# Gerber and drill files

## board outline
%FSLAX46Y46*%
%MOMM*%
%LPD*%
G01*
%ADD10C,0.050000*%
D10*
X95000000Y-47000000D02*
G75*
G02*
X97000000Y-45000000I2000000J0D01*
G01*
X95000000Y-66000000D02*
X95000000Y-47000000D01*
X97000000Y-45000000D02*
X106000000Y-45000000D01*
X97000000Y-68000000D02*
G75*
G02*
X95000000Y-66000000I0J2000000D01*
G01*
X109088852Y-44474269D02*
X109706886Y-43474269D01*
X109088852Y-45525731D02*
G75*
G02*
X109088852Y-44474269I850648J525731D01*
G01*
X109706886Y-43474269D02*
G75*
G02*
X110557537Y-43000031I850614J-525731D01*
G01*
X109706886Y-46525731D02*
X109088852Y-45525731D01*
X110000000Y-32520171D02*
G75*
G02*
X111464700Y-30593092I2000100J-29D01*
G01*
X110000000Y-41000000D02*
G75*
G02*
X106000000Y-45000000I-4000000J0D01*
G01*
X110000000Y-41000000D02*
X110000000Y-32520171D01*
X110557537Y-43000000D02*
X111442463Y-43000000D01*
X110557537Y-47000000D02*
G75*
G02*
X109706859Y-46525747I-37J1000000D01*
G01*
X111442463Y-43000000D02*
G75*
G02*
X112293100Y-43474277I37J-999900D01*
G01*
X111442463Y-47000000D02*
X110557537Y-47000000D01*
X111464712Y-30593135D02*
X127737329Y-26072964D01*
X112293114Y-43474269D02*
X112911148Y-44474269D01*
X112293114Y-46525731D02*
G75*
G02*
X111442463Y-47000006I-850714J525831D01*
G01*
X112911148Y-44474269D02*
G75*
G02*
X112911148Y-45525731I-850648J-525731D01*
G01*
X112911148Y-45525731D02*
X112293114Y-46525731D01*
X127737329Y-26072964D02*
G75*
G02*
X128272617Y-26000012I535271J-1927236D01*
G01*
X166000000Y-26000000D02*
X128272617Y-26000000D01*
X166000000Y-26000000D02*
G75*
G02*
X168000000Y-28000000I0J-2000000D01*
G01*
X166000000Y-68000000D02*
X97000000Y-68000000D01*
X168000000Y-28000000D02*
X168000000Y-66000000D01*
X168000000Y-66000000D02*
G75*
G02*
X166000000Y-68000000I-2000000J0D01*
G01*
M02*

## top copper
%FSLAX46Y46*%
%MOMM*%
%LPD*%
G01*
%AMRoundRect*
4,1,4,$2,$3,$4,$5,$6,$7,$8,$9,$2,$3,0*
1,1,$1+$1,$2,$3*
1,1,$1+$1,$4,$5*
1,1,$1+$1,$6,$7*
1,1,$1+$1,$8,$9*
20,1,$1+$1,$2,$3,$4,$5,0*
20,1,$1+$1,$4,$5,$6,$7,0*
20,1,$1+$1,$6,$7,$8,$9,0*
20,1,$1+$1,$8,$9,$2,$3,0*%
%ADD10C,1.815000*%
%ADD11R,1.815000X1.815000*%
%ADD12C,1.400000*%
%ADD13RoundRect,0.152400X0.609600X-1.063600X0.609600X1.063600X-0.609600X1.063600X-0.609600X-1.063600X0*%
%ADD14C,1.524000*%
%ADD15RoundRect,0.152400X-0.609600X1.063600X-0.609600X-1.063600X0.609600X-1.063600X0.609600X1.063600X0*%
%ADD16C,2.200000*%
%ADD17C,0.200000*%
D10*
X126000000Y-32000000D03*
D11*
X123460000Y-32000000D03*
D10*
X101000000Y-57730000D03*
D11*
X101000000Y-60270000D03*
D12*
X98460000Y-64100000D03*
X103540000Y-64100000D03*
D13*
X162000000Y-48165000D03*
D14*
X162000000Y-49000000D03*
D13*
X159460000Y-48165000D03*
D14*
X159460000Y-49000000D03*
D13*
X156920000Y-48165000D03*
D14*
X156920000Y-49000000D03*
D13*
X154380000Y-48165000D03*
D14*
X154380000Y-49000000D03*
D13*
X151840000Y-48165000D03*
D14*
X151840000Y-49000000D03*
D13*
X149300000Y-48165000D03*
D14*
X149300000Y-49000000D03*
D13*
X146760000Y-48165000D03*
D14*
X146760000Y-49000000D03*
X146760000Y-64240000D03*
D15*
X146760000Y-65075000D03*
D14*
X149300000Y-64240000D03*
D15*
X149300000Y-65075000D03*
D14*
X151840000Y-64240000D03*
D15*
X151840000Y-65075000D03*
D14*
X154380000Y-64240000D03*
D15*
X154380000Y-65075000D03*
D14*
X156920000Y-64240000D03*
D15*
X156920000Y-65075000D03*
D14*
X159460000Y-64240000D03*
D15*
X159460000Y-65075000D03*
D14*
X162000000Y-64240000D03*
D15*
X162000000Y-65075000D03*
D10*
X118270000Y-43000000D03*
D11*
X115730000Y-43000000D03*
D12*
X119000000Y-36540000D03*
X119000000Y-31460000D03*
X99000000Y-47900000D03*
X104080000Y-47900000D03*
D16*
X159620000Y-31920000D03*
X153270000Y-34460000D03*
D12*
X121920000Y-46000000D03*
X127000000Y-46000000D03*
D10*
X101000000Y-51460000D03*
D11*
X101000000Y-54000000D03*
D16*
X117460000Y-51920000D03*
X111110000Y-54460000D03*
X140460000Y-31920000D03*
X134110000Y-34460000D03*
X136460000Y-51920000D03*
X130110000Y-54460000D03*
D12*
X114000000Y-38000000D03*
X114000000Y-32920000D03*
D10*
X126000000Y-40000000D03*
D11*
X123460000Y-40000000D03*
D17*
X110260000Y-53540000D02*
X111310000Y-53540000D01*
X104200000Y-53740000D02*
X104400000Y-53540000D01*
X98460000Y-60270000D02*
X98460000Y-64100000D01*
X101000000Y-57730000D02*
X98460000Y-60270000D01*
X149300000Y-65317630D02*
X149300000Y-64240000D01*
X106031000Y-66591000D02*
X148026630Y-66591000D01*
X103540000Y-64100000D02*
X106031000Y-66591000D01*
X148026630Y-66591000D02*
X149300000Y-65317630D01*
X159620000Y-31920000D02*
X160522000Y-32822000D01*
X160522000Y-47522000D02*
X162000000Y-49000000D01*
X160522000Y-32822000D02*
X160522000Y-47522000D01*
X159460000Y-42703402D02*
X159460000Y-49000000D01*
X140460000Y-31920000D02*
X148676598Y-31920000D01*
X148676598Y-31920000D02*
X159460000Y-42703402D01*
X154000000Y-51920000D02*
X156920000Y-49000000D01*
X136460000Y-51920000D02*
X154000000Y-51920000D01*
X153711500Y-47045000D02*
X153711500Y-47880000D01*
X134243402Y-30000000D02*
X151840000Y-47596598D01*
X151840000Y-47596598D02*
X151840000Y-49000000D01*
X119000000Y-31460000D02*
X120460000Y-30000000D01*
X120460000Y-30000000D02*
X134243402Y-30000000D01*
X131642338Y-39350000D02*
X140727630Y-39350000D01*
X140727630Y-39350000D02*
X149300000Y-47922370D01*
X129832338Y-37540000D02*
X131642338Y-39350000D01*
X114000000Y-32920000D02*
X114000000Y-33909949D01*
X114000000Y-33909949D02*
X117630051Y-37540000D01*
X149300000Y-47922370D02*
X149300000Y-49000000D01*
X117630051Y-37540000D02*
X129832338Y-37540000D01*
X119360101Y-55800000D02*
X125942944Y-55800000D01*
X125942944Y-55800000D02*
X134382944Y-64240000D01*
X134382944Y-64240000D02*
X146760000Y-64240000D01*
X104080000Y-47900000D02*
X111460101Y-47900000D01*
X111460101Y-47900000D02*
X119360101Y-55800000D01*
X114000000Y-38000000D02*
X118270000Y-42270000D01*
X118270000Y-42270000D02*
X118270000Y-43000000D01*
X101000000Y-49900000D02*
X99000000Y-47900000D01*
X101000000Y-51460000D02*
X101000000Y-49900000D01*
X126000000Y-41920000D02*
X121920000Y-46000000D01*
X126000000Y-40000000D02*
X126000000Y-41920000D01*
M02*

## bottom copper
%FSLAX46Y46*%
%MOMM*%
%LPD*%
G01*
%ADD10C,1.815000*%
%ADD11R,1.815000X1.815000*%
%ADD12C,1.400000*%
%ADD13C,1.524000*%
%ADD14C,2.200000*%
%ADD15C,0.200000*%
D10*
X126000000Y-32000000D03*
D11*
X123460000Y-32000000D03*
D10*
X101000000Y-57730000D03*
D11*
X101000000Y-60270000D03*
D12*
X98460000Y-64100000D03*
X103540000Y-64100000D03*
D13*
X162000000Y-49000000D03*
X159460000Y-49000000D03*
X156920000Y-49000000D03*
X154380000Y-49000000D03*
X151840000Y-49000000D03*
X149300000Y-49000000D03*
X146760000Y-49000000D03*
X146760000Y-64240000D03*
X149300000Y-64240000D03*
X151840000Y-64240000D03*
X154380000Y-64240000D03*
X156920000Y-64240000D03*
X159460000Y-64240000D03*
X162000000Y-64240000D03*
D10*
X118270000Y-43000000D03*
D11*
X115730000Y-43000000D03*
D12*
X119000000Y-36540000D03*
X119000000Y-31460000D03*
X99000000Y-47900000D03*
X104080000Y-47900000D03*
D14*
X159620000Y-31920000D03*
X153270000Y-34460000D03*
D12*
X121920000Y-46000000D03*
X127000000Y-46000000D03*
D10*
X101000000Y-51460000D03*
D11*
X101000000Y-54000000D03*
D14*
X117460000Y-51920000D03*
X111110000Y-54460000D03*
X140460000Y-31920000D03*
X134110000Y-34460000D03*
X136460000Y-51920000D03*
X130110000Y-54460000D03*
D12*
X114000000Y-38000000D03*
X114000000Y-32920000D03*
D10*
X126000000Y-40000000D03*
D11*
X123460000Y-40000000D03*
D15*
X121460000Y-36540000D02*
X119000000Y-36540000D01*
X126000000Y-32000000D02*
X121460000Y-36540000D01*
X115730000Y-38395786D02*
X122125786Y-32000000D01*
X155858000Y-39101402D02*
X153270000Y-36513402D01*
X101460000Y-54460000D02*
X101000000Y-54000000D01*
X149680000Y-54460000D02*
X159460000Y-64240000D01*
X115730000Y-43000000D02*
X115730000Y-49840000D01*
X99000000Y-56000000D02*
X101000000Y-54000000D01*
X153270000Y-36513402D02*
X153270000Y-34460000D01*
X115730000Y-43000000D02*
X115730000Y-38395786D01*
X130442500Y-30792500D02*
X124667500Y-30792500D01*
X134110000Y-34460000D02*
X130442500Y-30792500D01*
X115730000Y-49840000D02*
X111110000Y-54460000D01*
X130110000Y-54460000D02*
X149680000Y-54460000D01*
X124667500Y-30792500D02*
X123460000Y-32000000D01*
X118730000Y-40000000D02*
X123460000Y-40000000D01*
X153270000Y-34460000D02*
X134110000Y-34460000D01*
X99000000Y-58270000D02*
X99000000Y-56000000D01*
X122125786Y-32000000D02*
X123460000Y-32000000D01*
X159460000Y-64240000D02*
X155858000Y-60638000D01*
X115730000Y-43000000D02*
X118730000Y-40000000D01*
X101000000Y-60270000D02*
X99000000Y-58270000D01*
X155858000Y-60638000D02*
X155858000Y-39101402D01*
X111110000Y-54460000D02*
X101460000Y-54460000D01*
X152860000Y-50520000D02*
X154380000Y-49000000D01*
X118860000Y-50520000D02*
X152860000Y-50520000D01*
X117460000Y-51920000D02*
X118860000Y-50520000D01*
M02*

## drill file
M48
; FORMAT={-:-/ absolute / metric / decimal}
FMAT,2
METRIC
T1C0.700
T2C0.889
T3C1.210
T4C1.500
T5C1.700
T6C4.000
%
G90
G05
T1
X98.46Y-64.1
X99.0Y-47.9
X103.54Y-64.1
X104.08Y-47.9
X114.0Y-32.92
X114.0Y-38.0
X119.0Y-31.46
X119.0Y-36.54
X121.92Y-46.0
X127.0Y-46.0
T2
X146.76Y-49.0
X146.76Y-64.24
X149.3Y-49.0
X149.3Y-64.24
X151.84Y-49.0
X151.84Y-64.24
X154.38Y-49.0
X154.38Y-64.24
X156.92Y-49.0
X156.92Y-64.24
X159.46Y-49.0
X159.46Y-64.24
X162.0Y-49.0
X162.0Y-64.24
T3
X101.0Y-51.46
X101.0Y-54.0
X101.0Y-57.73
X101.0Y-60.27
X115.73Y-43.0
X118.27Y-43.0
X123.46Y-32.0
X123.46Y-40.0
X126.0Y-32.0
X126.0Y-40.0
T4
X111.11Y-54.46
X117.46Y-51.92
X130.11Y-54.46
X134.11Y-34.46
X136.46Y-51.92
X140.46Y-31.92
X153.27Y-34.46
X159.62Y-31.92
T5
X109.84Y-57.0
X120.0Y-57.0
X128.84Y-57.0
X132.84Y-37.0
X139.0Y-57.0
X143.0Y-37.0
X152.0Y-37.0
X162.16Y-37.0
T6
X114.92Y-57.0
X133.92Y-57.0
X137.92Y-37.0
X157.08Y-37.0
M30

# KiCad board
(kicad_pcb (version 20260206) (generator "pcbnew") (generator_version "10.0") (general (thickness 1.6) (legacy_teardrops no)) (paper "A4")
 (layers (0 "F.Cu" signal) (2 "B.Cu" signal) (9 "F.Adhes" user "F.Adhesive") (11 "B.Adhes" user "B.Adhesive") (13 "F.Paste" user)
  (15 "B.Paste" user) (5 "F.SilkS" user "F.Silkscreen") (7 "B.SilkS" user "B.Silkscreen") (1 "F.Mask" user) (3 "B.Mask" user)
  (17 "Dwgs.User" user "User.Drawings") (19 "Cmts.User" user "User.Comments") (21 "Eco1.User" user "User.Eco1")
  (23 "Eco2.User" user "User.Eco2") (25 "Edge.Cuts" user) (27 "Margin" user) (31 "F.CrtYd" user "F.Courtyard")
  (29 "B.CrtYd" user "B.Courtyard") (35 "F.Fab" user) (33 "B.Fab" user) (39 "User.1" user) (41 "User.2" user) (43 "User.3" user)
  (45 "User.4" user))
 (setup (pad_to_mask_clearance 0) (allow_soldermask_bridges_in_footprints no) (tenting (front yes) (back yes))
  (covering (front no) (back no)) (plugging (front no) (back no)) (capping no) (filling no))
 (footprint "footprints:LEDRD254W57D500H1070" (layer "F.Cu") (at 124.73 32)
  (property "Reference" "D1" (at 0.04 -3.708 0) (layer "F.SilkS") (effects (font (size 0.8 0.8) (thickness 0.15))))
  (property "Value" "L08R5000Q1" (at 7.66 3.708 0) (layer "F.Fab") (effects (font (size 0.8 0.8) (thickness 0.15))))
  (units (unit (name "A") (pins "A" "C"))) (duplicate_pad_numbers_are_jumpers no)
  (pad "A" thru_hole circle (at 1.27 0) (size 1.815 1.815) (drill 1.21) (layers "*.Cu" "*.Mask") (remove_unused_layers no)
   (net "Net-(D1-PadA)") (solder_mask_margin 0.102))
  (pad "C" thru_hole rect (at -1.27 0) (size 1.815 1.815) (drill 1.21) (layers "*.Cu" "*.Mask") (remove_unused_layers no) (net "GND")
   (solder_mask_margin 0.102)))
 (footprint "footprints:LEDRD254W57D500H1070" (layer "F.Cu") (at 101 59 90)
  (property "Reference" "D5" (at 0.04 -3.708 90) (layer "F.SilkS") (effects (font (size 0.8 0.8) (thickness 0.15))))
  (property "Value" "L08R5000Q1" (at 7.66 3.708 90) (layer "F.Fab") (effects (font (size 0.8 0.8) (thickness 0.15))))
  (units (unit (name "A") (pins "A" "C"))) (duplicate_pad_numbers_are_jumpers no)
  (pad "A" thru_hole circle (at 1.27 0 90) (size 1.815 1.815) (drill 1.21) (layers "*.Cu" "*.Mask") (remove_unused_layers no)
   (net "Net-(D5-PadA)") (solder_mask_margin 0.102))
  (pad "C" thru_hole rect (at -1.27 0 90) (size 1.815 1.815) (drill 1.21) (layers "*.Cu" "*.Mask") (remove_unused_layers no) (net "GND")
   (solder_mask_margin 0.102)))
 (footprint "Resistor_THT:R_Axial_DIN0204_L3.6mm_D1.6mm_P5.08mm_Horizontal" (layer "F.Cu") (at 98.46 64.1)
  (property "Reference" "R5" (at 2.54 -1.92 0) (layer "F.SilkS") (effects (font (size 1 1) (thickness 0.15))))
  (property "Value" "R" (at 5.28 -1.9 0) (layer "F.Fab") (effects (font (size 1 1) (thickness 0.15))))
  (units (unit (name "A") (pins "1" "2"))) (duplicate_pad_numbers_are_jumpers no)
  (pad "1" thru_hole circle (at 0 0) (size 1.4 1.4) (drill 0.7) (layers "*.Cu" "*.Mask") (remove_unused_layers no) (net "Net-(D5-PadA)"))
  (pad "2" thru_hole circle (at 5.08 0) (size 1.4 1.4) (drill 0.7) (layers "*.Cu" "*.Mask") (remove_unused_layers no) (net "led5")))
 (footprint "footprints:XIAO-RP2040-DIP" (layer "F.Cu") (at 154.38 56.62)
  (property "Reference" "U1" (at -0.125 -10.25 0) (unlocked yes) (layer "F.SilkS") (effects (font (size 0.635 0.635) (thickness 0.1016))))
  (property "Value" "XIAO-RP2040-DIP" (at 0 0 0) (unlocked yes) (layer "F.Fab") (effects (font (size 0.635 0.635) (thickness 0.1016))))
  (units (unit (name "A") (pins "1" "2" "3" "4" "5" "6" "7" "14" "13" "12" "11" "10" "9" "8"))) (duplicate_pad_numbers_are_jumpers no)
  (pad "1" smd roundrect (at 7.62 -8.455 90) (size 2.432 1.524) (layers "F.Cu" "F.Mask") (roundrect_rratio 0.1) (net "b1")
   (thermal_bridge_angle 45))
  (pad "1" thru_hole circle (at 7.62 -7.62 90) (size 1.524 1.524) (drill 0.889) (layers "*.Cu" "*.Mask") (remove_unused_layers no)
   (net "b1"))
  (pad "2" smd roundrect (at 5.08 -8.455 90) (size 2.432 1.524) (layers "F.Cu" "F.Mask") (roundrect_rratio 0.1) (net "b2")
   (thermal_bridge_angle 45))
  (pad "2" thru_hole circle (at 5.08 -7.62 90) (size 1.524 1.524) (drill 0.889) (layers "*.Cu" "*.Mask") (remove_unused_layers no)
   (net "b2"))
  (pad "3" smd roundrect (at 2.54 -8.455 90) (size 2.432 1.524) (layers "F.Cu" "F.Mask") (roundrect_rratio 0.1) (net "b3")
   (thermal_bridge_angle 45))
  (pad "3" thru_hole circle (at 2.54 -7.62 90) (size 1.524 1.524) (drill 0.889) (layers "*.Cu" "*.Mask") (remove_unused_layers no)
   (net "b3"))
  (pad "4" smd roundrect (at 0 -8.455 90) (size 2.432 1.524) (layers "F.Cu" "F.Mask") (roundrect_rratio 0.1) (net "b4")
   (thermal_bridge_angle 45))
  (pad "4" thru_hole circle (at 0 -7.62 90) (size 1.524 1.524) (drill 0.889) (layers "*.Cu" "*.Mask") (remove_unused_layers no) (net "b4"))
  (pad "5" smd roundrect (at -2.54 -8.455 90) (size 2.432 1.524) (layers "F.Cu" "F.Mask") (roundrect_rratio 0.1) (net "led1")
   (thermal_bridge_angle 45))
  (pad "5" thru_hole circle (at -2.54 -7.62 90) (size 1.524 1.524) (drill 0.889) (layers "*.Cu" "*.Mask") (remove_unused_layers no)
   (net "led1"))
  (pad "6" smd roundrect (at -5.08 -8.455 90) (size 2.432 1.524) (layers "F.Cu" "F.Mask") (roundrect_rratio 0.1) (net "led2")
   (thermal_bridge_angle 45))
  (pad "6" thru_hole circle (at -5.08 -7.62 90) (size 1.524 1.524) (drill 0.889) (layers "*.Cu" "*.Mask") (remove_unused_layers no)
   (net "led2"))
  (pad "7" smd roundrect (at -7.62 -8.455 90) (size 2.432 1.524) (layers "F.Cu" "F.Mask") (roundrect_rratio 0.1) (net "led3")
   (thermal_bridge_angle 45))
  (pad "7" thru_hole circle (at -7.62 -7.62 90) (size 1.524 1.524) (drill 0.889) (layers "*.Cu" "*.Mask") (remove_unused_layers no)
   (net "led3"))
  (pad "8" thru_hole circle (at -7.62 7.62 270) (size 1.524 1.524) (drill 0.889) (layers "*.Cu" "*.Mask") (remove_unused_layers no)
   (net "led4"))
  (pad "8" smd roundrect (at -7.62 8.455 270) (size 2.432 1.524) (layers "F.Cu" "F.Mask") (roundrect_rratio 0.1) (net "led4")
   (thermal_bridge_angle 45))
  (pad "9" thru_hole circle (at -5.08 7.62 270) (size 1.524 1.524) (drill 0.889) (layers "*.Cu" "*.Mask") (remove_unused_layers no)
   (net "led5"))
  (pad "9" smd roundrect (at -5.08 8.455 270) (size 2.432 1.524) (layers "F.Cu" "F.Mask") (roundrect_rratio 0.1) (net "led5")
   (thermal_bridge_angle 45))
  (pad "10" thru_hole circle (at -2.54 7.62 270) (size 1.524 1.524) (drill 0.889) (layers "*.Cu" "*.Mask") (remove_unused_layers no)
   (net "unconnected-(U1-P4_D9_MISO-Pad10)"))
  (pad "10" smd roundrect (at -2.54 8.455 270) (size 2.432 1.524) (layers "F.Cu" "F.Mask") (roundrect_rratio 0.1)
   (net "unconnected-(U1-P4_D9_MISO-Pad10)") (thermal_bridge_angle 45))
  (pad "11" thru_hole circle (at 0 7.62 270) (size 1.524 1.524) (drill 0.889) (layers "*.Cu" "*.Mask") (remove_unused_layers no)
   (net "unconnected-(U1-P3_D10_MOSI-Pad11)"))
  (pad "11" smd roundrect (at 0 8.455 270) (size 2.432 1.524) (layers "F.Cu" "F.Mask") (roundrect_rratio 0.1)
   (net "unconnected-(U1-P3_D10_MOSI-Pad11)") (thermal_bridge_angle 45))
  (pad "12" thru_hole circle (at 2.54 7.62 270) (size 1.524 1.524) (drill 0.889) (layers "*.Cu" "*.Mask") (remove_unused_layers no)
   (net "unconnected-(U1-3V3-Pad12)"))
  (pad "12" smd roundrect (at 2.54 8.455 270) (size 2.432 1.524) (layers "F.Cu" "F.Mask") (roundrect_rratio 0.1)
   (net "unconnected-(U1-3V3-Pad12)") (thermal_bridge_angle 45))
  (pad "13" thru_hole circle (at 5.08 7.62 270) (size 1.524 1.524) (drill 0.889) (layers "*.Cu" "*.Mask") (remove_unused_layers no)
   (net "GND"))
  (pad "13" smd roundrect (at 5.08 8.455 270) (size 2.432 1.524) (layers "F.Cu" "F.Mask") (roundrect_rratio 0.1) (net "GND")
   (thermal_bridge_angle 45))
  (pad "14" thru_hole circle (at 7.62 7.62 270) (size 1.524 1.524) (drill 0.889) (layers "*.Cu" "*.Mask") (remove_unused_layers no)
   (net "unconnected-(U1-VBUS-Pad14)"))
  (pad "14" smd roundrect (at 7.62 8.455 270) (size 2.432 1.524) (layers "F.Cu" "F.Mask") (roundrect_rratio 0.1)
   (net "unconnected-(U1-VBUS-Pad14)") (thermal_bridge_angle 45)))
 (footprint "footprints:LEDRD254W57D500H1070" (layer "F.Cu") (at 117 43)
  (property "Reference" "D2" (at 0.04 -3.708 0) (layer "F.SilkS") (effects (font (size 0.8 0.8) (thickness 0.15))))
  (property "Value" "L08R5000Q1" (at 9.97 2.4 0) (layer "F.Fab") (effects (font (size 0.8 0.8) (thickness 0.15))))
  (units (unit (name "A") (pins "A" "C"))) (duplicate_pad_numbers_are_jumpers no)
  (pad "A" thru_hole circle (at 1.27 0) (size 1.815 1.815) (drill 1.21) (layers "*.Cu" "*.Mask") (remove_unused_layers no)
   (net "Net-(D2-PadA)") (solder_mask_margin 0.102))
  (pad "C" thru_hole rect (at -1.27 0) (size 1.815 1.815) (drill 1.21) (layers "*.Cu" "*.Mask") (remove_unused_layers no) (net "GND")
   (solder_mask_margin 0.102)))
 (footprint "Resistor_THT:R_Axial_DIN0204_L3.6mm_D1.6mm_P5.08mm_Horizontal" (layer "F.Cu") (at 119 36.54 90)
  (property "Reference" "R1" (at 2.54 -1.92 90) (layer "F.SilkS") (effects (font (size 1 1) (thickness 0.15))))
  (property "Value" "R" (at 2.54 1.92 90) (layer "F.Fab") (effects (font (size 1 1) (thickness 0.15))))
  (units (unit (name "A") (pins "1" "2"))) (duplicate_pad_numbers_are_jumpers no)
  (pad "1" thru_hole circle (at 0 0 90) (size 1.4 1.4) (drill 0.7) (layers "*.Cu" "*.Mask") (remove_unused_layers no) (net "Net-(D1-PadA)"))
  (pad "2" thru_hole circle (at 5.08 0 90) (size 1.4 1.4) (drill 0.7) (layers "*.Cu" "*.Mask") (remove_unused_layers no) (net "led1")))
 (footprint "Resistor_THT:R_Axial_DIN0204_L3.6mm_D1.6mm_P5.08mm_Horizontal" (layer "F.Cu") (at 99 47.9)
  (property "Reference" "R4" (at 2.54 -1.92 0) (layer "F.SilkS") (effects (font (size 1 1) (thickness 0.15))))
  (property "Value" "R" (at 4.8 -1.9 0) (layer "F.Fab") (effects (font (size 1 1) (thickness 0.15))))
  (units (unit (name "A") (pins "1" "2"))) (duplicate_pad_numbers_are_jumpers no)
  (pad "1" thru_hole circle (at 0 0) (size 1.4 1.4) (drill 0.7) (layers "*.Cu" "*.Mask") (remove_unused_layers no) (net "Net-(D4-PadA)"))
  (pad "2" thru_hole circle (at 5.08 0) (size 1.4 1.4) (drill 0.7) (layers "*.Cu" "*.Mask") (remove_unused_layers no) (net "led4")))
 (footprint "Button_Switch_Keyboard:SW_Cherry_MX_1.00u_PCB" (layer "F.Cu") (at 159.62 31.92)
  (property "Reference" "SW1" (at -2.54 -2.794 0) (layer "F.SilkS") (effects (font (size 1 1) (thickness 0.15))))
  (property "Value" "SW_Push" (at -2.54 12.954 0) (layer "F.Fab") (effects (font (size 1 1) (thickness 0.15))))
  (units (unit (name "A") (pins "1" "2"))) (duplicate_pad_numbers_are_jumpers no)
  (pad "" np_thru_hole circle (at -7.62 5.08) (size 1.7 1.7) (drill 1.7) (layers "*.Cu" "*.Mask"))
  (pad "" np_thru_hole circle (at -2.54 5.08) (size 4 4) (drill 4) (layers "*.Cu" "*.Mask"))
  (pad "" np_thru_hole circle (at 2.54 5.08) (size 1.7 1.7) (drill 1.7) (layers "*.Cu" "*.Mask"))
  (pad "1" thru_hole circle (at 0 0) (size 2.2 2.2) (drill 1.5) (layers "*.Cu" "*.Mask") (remove_unused_layers no) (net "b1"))
  (pad "2" thru_hole circle (at -6.35 2.54) (size 2.2 2.2) (drill 1.5) (layers "*.Cu" "*.Mask") (remove_unused_layers no) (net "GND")))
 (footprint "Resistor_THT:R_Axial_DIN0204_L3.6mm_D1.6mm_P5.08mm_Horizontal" (layer "F.Cu") (at 121.92 46)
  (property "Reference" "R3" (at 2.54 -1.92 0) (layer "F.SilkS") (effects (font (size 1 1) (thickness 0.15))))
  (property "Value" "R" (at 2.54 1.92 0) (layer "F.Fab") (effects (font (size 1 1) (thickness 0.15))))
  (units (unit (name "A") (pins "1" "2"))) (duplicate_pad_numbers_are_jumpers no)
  (pad "1" thru_hole circle (at 0 0) (size 1.4 1.4) (drill 0.7) (layers "*.Cu" "*.Mask") (remove_unused_layers no) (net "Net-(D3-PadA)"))
  (pad "2" thru_hole circle (at 5.08 0) (size 1.4 1.4) (drill 0.7) (layers "*.Cu" "*.Mask") (remove_unused_layers no) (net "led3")))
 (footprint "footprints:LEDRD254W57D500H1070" (layer "F.Cu") (at 101 52.73 90)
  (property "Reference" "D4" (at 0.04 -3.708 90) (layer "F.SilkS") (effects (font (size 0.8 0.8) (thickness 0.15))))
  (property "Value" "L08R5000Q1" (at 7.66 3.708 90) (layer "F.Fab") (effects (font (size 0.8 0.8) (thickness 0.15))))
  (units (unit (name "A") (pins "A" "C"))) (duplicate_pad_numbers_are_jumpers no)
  (pad "A" thru_hole circle (at 1.27 0 90) (size 1.815 1.815) (drill 1.21) (layers "*.Cu" "*.Mask") (remove_unused_layers no)
   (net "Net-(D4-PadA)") (solder_mask_margin 0.102))
  (pad "C" thru_hole rect (at -1.27 0 90) (size 1.815 1.815) (drill 1.21) (layers "*.Cu" "*.Mask") (remove_unused_layers no) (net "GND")
   (solder_mask_margin 0.102)))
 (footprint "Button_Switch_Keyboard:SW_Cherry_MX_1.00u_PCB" (layer "F.Cu") (at 117.46 51.92)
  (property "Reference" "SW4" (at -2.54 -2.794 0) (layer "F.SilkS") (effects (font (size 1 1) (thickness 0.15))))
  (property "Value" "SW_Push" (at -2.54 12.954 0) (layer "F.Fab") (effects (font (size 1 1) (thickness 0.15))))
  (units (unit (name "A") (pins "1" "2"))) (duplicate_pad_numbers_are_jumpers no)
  (pad "" np_thru_hole circle (at -7.62 5.08) (size 1.7 1.7) (drill 1.7) (layers "*.Cu" "*.Mask"))
  (pad "" np_thru_hole circle (at -2.54 5.08) (size 4 4) (drill 4) (layers "*.Cu" "*.Mask"))
  (pad "" np_thru_hole circle (at 2.54 5.08) (size 1.7 1.7) (drill 1.7) (layers "*.Cu" "*.Mask"))
  (pad "1" thru_hole circle (at 0 0) (size 2.2 2.2) (drill 1.5) (layers "*.Cu" "*.Mask") (remove_unused_layers no) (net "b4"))
  (pad "2" thru_hole circle (at -6.35 2.54) (size 2.2 2.2) (drill 1.5) (layers "*.Cu" "*.Mask") (remove_unused_layers no) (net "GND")))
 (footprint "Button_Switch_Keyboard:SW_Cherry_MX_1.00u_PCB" (layer "F.Cu") (at 140.46 31.92)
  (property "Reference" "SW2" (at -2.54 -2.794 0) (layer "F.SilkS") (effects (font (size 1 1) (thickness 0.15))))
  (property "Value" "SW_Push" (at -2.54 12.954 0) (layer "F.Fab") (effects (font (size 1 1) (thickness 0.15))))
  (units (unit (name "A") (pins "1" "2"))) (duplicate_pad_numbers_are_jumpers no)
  (pad "" np_thru_hole circle (at -7.62 5.08) (size 1.7 1.7) (drill 1.7) (layers "*.Cu" "*.Mask"))
  (pad "" np_thru_hole circle (at -2.54 5.08) (size 4 4) (drill 4) (layers "*.Cu" "*.Mask"))
  (pad "" np_thru_hole circle (at 2.54 5.08) (size 1.7 1.7) (drill 1.7) (layers "*.Cu" "*.Mask"))
  (pad "1" thru_hole circle (at 0 0) (size 2.2 2.2) (drill 1.5) (layers "*.Cu" "*.Mask") (remove_unused_layers no) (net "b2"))
  (pad "2" thru_hole circle (at -6.35 2.54) (size 2.2 2.2) (drill 1.5) (layers "*.Cu" "*.Mask") (remove_unused_layers no) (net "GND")))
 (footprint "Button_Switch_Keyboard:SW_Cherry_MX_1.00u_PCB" (layer "F.Cu") (at 136.46 51.92)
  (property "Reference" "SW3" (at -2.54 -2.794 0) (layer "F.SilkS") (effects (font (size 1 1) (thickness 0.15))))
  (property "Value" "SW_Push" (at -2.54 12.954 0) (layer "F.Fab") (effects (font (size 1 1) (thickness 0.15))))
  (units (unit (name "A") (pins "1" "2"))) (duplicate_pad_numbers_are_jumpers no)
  (pad "" np_thru_hole circle (at -7.62 5.08) (size 1.7 1.7) (drill 1.7) (layers "*.Cu" "*.Mask"))
  (pad "" np_thru_hole circle (at -2.54 5.08) (size 4 4) (drill 4) (layers "*.Cu" "*.Mask"))
  (pad "" np_thru_hole circle (at 2.54 5.08) (size 1.7 1.7) (drill 1.7) (layers "*.Cu" "*.Mask"))
  (pad "1" thru_hole circle (at 0 0) (size 2.2 2.2) (drill 1.5) (layers "*.Cu" "*.Mask") (remove_unused_layers no) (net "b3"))
  (pad "2" thru_hole circle (at -6.35 2.54) (size 2.2 2.2) (drill 1.5) (layers "*.Cu" "*.Mask") (remove_unused_layers no) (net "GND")))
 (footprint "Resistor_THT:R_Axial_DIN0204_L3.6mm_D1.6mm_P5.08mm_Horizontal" (layer "F.Cu") (at 114 38 90)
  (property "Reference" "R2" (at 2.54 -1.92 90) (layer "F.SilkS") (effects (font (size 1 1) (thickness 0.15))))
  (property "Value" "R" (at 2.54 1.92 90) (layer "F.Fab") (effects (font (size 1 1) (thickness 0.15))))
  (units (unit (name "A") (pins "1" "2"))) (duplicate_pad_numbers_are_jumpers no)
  (pad "1" thru_hole circle (at 0 0 90) (size 1.4 1.4) (drill 0.7) (layers "*.Cu" "*.Mask") (remove_unused_layers no) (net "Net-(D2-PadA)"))
  (pad "2" thru_hole circle (at 5.08 0 90) (size 1.4 1.4) (drill 0.7) (layers "*.Cu" "*.Mask") (remove_unused_layers no) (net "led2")))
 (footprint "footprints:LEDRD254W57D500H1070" (layer "F.Cu") (at 124.73 40)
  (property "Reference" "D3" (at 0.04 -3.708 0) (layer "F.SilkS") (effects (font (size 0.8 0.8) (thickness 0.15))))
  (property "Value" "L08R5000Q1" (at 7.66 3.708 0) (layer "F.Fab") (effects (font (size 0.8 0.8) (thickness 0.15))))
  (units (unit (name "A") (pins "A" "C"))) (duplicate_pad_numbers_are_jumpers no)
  (pad "A" thru_hole circle (at 1.27 0) (size 1.815 1.815) (drill 1.21) (layers "*.Cu" "*.Mask") (remove_unused_layers no)
   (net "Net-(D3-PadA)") (solder_mask_margin 0.102))
  (pad "C" thru_hole rect (at -1.27 0) (size 1.815 1.815) (drill 1.21) (layers "*.Cu" "*.Mask") (remove_unused_layers no) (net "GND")
   (solder_mask_margin 0.102)))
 (gr_arc (start 95 47) (mid 95.585786 45.585786) (end 97 45) (stroke (width 0.05) (type default)) (layer "Edge.Cuts"))
 (gr_line (start 95 66) (end 95 47) (stroke (width 0.05) (type default)) (layer "Edge.Cuts"))
 (gr_line (start 97 45) (end 106 45) (stroke (width 0.05) (type default)) (layer "Edge.Cuts"))
 (gr_arc (start 97 68) (mid 95.585786 67.414214) (end 95 66) (stroke (width 0.05) (type default)) (layer "Edge.Cuts"))
 (gr_line (start 109.088852 44.474269) (end 109.706886 43.474269) (stroke (width 0.05) (type default)) (layer "Edge.Cuts"))
 (gr_arc (start 109.088852 45.525731) (mid 108.939503 45) (end 109.088852 44.474269) (stroke (width 0.05) (type default))
  (layer "Edge.Cuts"))
 (gr_arc (start 109.706886 43.474269) (mid 110.070572 43.126578) (end 110.557537 43) (stroke (width 0.05) (type default))
  (layer "Edge.Cuts"))
 (gr_line (start 109.706886 46.525731) (end 109.088852 45.525731) (stroke (width 0.05) (type default)) (layer "Edge.Cuts"))
 (gr_arc (start 110 32.520171) (mid 110.407752 31.309932) (end 111.464712 30.593135) (stroke (width 0.05) (type default))
  (layer "Edge.Cuts"))
 (gr_arc (start 110 41) (mid 108.828427 43.828427) (end 106 45) (stroke (width 0.05) (type default)) (layer "Edge.Cuts"))
 (gr_line (start 110 41) (end 110 32.520171) (stroke (width 0.05) (type default)) (layer "Edge.Cuts"))
 (gr_line (start 110.557537 43) (end 111.442463 43) (stroke (width 0.05) (type default)) (layer "Edge.Cuts"))
 (gr_arc (start 110.557537 47) (mid 110.070572 46.873422) (end 109.706886 46.525731) (stroke (width 0.05) (type default))
  (layer "Edge.Cuts"))
 (gr_arc (start 111.442463 43) (mid 111.92944 43.126565) (end 112.293114 43.474269) (stroke (width 0.05) (type default)) (layer "Edge.Cuts"))
 (gr_line (start 111.442463 47) (end 110.557537 47) (stroke (width 0.05) (type default)) (layer "Edge.Cuts"))
 (gr_line (start 111.464712 30.593135) (end 127.737329 26.072964) (stroke (width 0.05) (type default)) (layer "Edge.Cuts"))
 (gr_line (start 112.293114 43.474269) (end 112.911148 44.474269) (stroke (width 0.05) (type default)) (layer "Edge.Cuts"))
 (gr_arc (start 112.293114 46.525731) (mid 111.929425 46.873408) (end 111.442463 47) (stroke (width 0.05) (type default))
  (layer "Edge.Cuts"))
 (gr_arc (start 112.911148 44.474269) (mid 113.060497 45) (end 112.911148 45.525731) (stroke (width 0.05) (type default))
  (layer "Edge.Cuts"))
 (gr_line (start 112.911148 45.525731) (end 112.293114 46.525731) (stroke (width 0.05) (type default)) (layer "Edge.Cuts"))
 (gr_arc (start 127.737329 26.072964) (mid 128.002498 26.018327) (end 128.272617 26) (stroke (width 0.05) (type default))
  (layer "Edge.Cuts"))
 (gr_line (start 166 26) (end 128.272617 26) (stroke (width 0.05) (type default)) (layer "Edge.Cuts"))
 (gr_arc (start 166 26) (mid 167.414214 26.585786) (end 168 28) (stroke (width 0.05) (type default)) (layer "Edge.Cuts"))
 (gr_line (start 166 68) (end 97 68) (stroke (width 0.05) (type default)) (layer "Edge.Cuts"))
 (gr_line (start 168 28) (end 168 66) (stroke (width 0.05) (type default)) (layer "Edge.Cuts"))
 (gr_arc (start 168 66) (mid 167.414214 67.414214) (end 166 68) (stroke (width 0.05) (type default)) (layer "Edge.Cuts"))
 (segment (start 121.46 36.54) (end 119 36.54) (width 0.2) (layer "B.Cu") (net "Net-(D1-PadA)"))
 (segment (start 126 32) (end 121.46 36.54) (width 0.2) (layer "B.Cu") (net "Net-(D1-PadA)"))
 (segment (start 110.26 53.54) (end 111.31 53.54) (width 0.2) (layer "F.Cu") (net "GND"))
 (segment (start 104.2 53.74) (end 104.4 53.54) (width 0.2) (layer "F.Cu") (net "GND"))
 (segment (start 115.73 38.395786) (end 122.125786 32) (width 0.2) (layer "B.Cu") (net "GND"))
 (segment (start 155.858 39.101402) (end 153.27 36.513402) (width 0.2) (layer "B.Cu") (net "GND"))
 (segment (start 101.46 54.46) (end 101 54) (width 0.2) (layer "B.Cu") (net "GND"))
 (segment (start 149.68 54.46) (end 159.46 64.24) (width 0.2) (layer "B.Cu") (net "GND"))
 (segment (start 115.73 43) (end 115.73 49.84) (width 0.2) (layer "B.Cu") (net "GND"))
 (segment (start 99 56) (end 101 54) (width 0.2) (layer "B.Cu") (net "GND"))
 (segment (start 153.27 36.513402) (end 153.27 34.46) (width 0.2) (layer "B.Cu") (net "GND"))
 (segment (start 115.73 43) (end 115.73 38.395786) (width 0.2) (layer "B.Cu") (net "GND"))
 (segment (start 130.4425 30.7925) (end 124.6675 30.7925) (width 0.2) (layer "B.Cu") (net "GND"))
 (segment (start 134.11 34.46) (end 130.4425 30.7925) (width 0.2) (layer "B.Cu") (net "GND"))
 (segment (start 115.73 49.84) (end 111.11 54.46) (width 0.2) (layer "B.Cu") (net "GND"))
 (segment (start 130.11 54.46) (end 149.68 54.46) (width 0.2) (layer "B.Cu") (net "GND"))
 (segment (start 124.6675 30.7925) (end 123.46 32) (width 0.2) (layer "B.Cu") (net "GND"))
 (segment (start 118.73 40) (end 123.46 40) (width 0.2) (layer "B.Cu") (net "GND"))
 (segment (start 153.27 34.46) (end 134.11 34.46) (width 0.2) (layer "B.Cu") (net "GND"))
 (segment (start 99 58.27) (end 99 56) (width 0.2) (layer "B.Cu") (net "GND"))
 (segment (start 122.125786 32) (end 123.46 32) (width 0.2) (layer "B.Cu") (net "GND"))
 (segment (start 159.46 64.24) (end 155.858 60.638) (width 0.2) (layer "B.Cu") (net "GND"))
 (segment (start 115.73 43) (end 118.73 40) (width 0.2) (layer "B.Cu") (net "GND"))
 (segment (start 101 60.27) (end 99 58.27) (width 0.2) (layer "B.Cu") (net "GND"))
 (segment (start 155.858 60.638) (end 155.858 39.101402) (width 0.2) (layer "B.Cu") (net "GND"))
 (segment (start 111.11 54.46) (end 101.46 54.46) (width 0.2) (layer "B.Cu") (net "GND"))
 (segment (start 98.46 60.27) (end 98.46 64.1) (width 0.2) (layer "F.Cu") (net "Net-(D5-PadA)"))
 (segment (start 101 57.73) (end 98.46 60.27) (width 0.2) (layer "F.Cu") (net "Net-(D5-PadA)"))
 (segment (start 149.3 65.31763) (end 149.3 64.24) (width 0.2) (layer "F.Cu") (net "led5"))
 (segment (start 106.031 66.591) (end 148.02663 66.591) (width 0.2) (layer "F.Cu") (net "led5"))
 (segment (start 103.54 64.1) (end 106.031 66.591) (width 0.2) (layer "F.Cu") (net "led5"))
 (segment (start 148.02663 66.591) (end 149.3 65.31763) (width 0.2) (layer "F.Cu") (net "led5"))
 (segment (start 159.62 31.92) (end 160.522 32.822) (width 0.2) (layer "F.Cu") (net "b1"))
 (segment (start 160.522 47.522) (end 162 49) (width 0.2) (layer "F.Cu") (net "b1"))
 (segment (start 160.522 32.822) (end 160.522 47.522) (width 0.2) (layer "F.Cu") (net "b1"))
 (segment (start 159.46 42.703402) (end 159.46 49) (width 0.2) (layer "F.Cu") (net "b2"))
 (segment (start 140.46 31.92) (end 148.676598 31.92) (width 0.2) (layer "F.Cu") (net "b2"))
 (segment (start 148.676598 31.92) (end 159.46 42.703402) (width 0.2) (layer "F.Cu") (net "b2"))
 (segment (start 154 51.92) (end 156.92 49) (width 0.2) (layer "F.Cu") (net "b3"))
 (segment (start 136.46 51.92) (end 154 51.92) (width 0.2) (layer "F.Cu") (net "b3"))
 (segment (start 153.7115 47.045) (end 153.7115 47.88) (width 0.2) (layer "F.Cu") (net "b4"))
 (segment (start 152.86 50.52) (end 154.38 49) (width 0.2) (layer "B.Cu") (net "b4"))
 (segment (start 118.86 50.52) (end 152.86 50.52) (width 0.2) (layer "B.Cu") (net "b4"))
 (segment (start 117.46 51.92) (end 118.86 50.52) (width 0.2) (layer "B.Cu") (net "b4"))
 (segment (start 134.243402 30) (end 151.84 47.596598) (width 0.2) (layer "F.Cu") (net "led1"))
 (segment (start 151.84 47.596598) (end 151.84 49) (width 0.2) (layer "F.Cu") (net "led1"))
 (segment (start 119 31.46) (end 120.46 30) (width 0.2) (layer "F.Cu") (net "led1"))
 (segment (start 120.46 30) (end 134.243402 30) (width 0.2) (layer "F.Cu") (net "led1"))
 (segment (start 131.642338 39.35) (end 140.72763 39.35) (width 0.2) (layer "F.Cu") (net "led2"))
 (segment (start 140.72763 39.35) (end 149.3 47.92237) (width 0.2) (layer "F.Cu") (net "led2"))
 (segment (start 129.832338 37.54) (end 131.642338 39.35) (width 0.2) (layer "F.Cu") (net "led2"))
 (segment (start 114 32.92) (end 114 33.909949) (width 0.2) (layer "F.Cu") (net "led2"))
 (segment (start 114 33.909949) (end 117.630051 37.54) (width 0.2) (layer "F.Cu") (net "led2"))
 (segment (start 149.3 47.92237) (end 149.3 49) (width 0.2) (layer "F.Cu") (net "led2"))
 (segment (start 117.630051 37.54) (end 129.832338 37.54) (width 0.2) (layer "F.Cu") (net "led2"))
 (segment (start 119.360101 55.8) (end 125.942944 55.8) (width 0.2) (layer "F.Cu") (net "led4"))
 (segment (start 125.942944 55.8) (end 134.382944 64.24) (width 0.2) (layer "F.Cu") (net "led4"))
 (segment (start 134.382944 64.24) (end 146.76 64.24) (width 0.2) (layer "F.Cu") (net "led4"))
 (segment (start 104.08 47.9) (end 111.460101 47.9) (width 0.2) (layer "F.Cu") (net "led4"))
 (segment (start 111.460101 47.9) (end 119.360101 55.8) (width 0.2) (layer "F.Cu") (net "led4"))
 (segment (start 114 38) (end 118.27 42.27) (width 0.2) (layer "F.Cu") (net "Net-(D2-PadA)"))
 (segment (start 118.27 42.27) (end 118.27 43) (width 0.2) (layer "F.Cu") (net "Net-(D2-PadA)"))
 (segment (start 101 49.9) (end 99 47.9) (width 0.2) (layer "F.Cu") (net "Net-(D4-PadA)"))
 (segment (start 101 51.46) (end 101 49.9) (width 0.2) (layer "F.Cu") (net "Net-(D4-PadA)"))
 (segment (start 126 41.92) (end 121.92 46) (width 0.2) (layer "F.Cu") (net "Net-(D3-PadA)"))
 (segment (start 126 40) (end 126 41.92) (width 0.2) (layer "F.Cu") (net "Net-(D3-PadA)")))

